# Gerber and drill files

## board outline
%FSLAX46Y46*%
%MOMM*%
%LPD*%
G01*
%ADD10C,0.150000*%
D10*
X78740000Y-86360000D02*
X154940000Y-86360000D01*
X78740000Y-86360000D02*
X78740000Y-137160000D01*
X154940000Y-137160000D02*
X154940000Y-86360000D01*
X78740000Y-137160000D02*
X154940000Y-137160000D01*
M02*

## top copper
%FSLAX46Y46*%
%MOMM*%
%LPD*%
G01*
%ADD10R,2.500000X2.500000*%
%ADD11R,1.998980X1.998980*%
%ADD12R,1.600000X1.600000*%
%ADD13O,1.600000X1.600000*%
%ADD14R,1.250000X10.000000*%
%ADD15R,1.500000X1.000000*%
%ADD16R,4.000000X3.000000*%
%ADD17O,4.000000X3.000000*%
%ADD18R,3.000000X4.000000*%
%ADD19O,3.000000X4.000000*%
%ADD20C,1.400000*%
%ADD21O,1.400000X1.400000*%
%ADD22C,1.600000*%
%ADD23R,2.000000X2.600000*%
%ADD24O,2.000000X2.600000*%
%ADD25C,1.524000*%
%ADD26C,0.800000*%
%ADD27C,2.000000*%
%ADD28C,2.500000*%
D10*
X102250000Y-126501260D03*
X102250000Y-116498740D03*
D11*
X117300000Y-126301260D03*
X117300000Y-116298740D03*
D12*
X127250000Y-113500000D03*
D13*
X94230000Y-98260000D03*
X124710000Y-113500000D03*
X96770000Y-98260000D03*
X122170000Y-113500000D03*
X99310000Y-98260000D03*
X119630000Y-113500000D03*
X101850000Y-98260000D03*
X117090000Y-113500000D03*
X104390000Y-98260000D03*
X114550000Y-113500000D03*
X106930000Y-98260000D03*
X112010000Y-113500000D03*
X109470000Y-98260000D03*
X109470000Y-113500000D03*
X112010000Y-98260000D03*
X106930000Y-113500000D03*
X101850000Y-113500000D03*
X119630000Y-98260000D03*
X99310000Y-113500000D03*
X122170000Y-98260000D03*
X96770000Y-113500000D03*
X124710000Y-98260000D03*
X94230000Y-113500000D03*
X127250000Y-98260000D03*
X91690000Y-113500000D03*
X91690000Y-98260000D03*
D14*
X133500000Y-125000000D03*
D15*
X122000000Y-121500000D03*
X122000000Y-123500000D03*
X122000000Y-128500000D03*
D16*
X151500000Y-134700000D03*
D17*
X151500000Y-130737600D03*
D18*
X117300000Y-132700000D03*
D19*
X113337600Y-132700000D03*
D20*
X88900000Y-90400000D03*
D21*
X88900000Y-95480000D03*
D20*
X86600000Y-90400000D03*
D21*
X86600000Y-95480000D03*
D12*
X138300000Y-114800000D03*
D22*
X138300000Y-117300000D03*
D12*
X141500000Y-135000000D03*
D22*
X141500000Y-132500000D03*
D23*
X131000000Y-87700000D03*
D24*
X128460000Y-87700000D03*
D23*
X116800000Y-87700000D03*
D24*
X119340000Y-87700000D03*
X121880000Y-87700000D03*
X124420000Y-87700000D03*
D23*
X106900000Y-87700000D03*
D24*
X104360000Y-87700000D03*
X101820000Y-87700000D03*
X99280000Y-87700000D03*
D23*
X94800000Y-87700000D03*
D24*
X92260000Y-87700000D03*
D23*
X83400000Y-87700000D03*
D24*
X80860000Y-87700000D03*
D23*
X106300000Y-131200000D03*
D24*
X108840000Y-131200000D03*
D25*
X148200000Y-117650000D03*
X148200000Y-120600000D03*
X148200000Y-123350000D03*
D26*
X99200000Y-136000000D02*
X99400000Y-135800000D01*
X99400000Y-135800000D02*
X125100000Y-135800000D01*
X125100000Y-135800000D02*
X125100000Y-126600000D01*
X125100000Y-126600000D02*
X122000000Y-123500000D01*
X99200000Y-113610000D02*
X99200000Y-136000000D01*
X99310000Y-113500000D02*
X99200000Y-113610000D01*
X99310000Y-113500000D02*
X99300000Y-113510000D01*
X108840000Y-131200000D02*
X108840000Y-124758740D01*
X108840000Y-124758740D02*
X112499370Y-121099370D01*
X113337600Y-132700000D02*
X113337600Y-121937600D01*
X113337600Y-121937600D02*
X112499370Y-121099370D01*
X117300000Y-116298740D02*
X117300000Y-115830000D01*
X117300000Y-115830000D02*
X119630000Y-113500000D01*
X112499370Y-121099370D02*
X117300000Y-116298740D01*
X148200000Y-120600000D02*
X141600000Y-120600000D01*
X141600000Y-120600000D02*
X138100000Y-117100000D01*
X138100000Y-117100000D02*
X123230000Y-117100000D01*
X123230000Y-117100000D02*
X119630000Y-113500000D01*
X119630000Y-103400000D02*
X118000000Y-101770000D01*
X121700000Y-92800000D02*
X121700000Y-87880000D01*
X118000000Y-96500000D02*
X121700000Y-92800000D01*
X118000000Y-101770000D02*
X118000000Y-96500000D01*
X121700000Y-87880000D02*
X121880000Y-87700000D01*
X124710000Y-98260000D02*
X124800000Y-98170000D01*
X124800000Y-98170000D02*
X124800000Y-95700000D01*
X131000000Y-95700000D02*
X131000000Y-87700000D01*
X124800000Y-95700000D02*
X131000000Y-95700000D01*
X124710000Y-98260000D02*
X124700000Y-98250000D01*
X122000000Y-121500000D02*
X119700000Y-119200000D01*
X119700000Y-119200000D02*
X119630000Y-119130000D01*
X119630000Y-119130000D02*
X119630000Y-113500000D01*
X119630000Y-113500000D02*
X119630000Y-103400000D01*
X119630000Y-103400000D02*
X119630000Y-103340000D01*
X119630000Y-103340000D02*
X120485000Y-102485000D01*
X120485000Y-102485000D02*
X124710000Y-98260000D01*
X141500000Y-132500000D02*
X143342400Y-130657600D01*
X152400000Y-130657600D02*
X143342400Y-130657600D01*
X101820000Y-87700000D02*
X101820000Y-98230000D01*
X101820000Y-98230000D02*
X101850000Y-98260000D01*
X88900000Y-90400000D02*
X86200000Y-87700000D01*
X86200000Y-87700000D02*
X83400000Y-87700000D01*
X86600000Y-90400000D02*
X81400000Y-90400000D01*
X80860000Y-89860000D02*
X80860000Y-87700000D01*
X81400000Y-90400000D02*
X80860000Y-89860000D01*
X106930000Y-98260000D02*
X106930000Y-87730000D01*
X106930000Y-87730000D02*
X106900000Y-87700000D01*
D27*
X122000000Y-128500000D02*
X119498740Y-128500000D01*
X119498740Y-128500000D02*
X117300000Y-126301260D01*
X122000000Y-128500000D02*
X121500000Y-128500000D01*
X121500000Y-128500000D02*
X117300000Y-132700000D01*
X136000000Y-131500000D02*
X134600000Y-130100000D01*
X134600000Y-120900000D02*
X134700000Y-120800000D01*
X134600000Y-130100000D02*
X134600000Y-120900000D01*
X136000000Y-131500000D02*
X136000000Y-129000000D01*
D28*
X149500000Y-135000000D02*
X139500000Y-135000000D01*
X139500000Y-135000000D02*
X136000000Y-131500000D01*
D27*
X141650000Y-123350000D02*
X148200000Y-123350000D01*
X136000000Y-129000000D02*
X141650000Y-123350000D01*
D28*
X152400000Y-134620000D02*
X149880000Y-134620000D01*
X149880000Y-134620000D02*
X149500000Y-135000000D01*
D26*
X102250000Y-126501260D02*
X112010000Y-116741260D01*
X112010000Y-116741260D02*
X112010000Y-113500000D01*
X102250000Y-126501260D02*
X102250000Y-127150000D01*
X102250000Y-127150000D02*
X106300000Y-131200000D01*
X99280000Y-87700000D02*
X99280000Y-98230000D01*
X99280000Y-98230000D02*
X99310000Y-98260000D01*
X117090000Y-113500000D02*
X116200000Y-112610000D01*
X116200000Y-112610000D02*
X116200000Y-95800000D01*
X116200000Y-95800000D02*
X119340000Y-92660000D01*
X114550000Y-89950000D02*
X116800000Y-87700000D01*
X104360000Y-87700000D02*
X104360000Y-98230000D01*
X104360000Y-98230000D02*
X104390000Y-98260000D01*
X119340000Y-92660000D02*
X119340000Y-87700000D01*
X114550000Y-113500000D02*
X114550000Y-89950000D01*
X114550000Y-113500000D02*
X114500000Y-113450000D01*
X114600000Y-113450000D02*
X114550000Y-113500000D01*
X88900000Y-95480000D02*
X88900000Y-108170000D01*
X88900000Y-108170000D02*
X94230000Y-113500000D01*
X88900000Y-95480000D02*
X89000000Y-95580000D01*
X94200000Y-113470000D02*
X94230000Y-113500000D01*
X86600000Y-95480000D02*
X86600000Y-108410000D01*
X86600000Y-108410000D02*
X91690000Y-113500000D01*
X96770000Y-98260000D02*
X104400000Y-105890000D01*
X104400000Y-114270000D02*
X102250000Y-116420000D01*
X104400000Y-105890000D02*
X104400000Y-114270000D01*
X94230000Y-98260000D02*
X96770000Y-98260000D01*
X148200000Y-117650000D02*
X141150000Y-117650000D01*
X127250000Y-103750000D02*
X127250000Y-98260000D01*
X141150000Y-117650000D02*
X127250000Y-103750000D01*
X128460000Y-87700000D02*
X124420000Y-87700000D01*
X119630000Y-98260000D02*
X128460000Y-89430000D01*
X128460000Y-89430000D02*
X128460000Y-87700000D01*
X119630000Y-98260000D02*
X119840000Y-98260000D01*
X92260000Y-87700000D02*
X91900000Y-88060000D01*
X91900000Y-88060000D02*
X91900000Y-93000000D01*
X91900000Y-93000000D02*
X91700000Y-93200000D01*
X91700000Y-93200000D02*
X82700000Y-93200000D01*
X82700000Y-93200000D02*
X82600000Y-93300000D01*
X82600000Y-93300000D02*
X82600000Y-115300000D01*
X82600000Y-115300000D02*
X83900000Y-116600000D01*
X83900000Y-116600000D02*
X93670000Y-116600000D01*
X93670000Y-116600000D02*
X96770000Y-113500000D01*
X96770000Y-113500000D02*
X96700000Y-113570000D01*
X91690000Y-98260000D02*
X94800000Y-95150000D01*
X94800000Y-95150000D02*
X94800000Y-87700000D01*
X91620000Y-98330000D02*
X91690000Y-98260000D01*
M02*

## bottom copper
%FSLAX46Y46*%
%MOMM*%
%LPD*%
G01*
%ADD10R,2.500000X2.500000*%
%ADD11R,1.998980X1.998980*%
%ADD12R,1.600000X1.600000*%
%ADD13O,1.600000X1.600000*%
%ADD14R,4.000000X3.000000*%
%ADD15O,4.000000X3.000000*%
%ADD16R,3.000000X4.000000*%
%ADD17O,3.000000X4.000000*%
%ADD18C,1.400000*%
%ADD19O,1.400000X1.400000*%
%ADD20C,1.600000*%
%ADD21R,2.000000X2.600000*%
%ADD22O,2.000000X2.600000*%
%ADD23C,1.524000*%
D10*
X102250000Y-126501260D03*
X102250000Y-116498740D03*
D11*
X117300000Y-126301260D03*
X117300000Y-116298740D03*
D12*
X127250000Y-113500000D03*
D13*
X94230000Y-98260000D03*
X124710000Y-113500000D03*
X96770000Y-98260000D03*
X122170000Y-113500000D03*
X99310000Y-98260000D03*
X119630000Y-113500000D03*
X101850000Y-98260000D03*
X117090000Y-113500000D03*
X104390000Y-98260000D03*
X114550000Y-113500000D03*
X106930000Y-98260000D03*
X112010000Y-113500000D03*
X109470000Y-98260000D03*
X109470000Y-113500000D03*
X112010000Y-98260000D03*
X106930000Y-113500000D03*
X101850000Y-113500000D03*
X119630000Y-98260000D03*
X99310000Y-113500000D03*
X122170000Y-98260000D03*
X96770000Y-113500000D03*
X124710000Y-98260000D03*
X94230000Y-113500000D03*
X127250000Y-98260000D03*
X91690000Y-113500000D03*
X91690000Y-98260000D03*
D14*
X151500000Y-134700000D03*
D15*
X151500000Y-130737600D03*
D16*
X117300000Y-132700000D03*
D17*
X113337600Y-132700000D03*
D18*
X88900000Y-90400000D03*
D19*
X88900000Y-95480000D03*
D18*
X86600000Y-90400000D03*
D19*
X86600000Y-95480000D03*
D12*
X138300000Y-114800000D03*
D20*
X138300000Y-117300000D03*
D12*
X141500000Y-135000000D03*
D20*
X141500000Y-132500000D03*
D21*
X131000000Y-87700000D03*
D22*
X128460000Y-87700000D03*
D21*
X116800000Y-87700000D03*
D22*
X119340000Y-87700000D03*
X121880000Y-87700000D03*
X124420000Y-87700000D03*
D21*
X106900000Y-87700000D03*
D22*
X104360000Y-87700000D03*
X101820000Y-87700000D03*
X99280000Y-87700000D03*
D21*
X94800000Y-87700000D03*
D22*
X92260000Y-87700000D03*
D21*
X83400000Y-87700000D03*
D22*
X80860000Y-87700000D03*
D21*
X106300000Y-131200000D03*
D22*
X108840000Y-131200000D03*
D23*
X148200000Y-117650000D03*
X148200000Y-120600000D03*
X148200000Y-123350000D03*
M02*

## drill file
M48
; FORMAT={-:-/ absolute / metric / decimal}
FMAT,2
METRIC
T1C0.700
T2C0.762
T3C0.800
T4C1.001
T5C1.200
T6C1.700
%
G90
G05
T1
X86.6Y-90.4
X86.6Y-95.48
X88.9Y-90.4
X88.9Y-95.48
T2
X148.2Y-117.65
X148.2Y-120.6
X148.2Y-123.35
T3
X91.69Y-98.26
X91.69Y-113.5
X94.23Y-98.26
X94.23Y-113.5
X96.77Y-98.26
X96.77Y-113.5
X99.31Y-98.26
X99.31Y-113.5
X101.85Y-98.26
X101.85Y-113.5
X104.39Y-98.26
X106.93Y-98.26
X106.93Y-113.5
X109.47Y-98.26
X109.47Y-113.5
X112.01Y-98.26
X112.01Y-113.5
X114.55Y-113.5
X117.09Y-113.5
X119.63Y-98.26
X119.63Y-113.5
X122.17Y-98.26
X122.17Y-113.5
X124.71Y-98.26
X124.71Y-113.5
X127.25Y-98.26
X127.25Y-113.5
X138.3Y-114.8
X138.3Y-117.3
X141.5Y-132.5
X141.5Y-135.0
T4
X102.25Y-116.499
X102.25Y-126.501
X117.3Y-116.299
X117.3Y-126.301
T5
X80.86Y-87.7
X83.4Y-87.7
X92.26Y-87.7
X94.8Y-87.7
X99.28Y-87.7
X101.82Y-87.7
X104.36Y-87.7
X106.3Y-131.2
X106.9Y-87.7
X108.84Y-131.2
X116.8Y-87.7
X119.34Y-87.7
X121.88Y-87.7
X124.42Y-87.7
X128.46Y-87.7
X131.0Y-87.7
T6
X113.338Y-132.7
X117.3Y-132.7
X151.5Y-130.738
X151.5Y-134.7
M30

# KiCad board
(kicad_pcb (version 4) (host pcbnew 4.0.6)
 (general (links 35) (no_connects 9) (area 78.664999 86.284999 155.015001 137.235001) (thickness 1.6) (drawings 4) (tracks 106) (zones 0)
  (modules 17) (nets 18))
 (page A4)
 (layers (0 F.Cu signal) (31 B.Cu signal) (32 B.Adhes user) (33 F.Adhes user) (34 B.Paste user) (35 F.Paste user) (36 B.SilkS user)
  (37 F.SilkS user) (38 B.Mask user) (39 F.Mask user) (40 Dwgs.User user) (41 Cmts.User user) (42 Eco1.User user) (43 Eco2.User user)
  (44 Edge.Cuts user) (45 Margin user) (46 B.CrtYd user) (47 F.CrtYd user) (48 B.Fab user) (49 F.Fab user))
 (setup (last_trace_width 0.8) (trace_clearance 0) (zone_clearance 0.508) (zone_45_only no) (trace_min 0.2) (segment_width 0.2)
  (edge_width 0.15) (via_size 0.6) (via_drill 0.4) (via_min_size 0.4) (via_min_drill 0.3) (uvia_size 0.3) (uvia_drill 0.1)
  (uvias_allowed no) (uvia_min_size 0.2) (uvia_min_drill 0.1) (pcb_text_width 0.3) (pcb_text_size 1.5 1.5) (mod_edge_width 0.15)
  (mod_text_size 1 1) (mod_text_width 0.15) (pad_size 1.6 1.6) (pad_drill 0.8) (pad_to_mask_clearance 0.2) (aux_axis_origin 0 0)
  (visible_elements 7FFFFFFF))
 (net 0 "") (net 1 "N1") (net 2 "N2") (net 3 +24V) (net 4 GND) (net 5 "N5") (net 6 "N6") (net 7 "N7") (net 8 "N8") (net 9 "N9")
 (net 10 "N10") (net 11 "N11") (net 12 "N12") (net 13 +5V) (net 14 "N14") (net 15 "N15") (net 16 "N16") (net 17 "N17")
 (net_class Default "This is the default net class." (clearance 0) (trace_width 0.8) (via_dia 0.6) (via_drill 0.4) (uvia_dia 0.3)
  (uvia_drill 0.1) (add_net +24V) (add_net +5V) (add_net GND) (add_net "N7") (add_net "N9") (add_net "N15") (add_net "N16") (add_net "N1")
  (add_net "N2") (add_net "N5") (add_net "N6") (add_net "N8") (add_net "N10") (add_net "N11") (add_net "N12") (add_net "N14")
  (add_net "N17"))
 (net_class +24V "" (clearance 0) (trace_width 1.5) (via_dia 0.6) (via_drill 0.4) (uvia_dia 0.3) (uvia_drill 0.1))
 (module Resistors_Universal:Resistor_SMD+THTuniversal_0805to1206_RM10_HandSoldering (layer F.Cu) (at 102.25 121.5 90)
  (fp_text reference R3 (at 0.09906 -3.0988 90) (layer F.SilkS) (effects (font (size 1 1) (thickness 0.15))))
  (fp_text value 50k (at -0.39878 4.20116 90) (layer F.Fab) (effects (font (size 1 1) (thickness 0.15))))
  (pad 1 thru_hole rect (at -5.00126 0 270) (size 2.5 2.5) (drill 1.00076) (layers *.Cu *.Mask) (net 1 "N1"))
  (pad 2 thru_hole rect (at 5.00126 0 270) (size 2.5 2.5) (drill 1.00076) (layers *.Cu *.Mask) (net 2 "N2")))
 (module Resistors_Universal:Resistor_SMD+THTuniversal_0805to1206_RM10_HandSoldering (layer F.Cu) (at 117.3 121.3 90)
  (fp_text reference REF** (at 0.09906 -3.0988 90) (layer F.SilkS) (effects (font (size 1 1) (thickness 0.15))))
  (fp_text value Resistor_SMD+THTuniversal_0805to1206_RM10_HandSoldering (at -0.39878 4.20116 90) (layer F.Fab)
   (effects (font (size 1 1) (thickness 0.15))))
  (pad 1 thru_hole rect (at -5.00126 0 270) (size 1.99898 1.99898) (drill 1.00076) (layers *.Cu *.Mask) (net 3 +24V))
  (pad "" thru_hole rect (at 5.00126 0 270) (size 1.99898 1.99898) (drill 1.00076) (layers *.Cu *.Mask) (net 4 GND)))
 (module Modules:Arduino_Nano (layer B.Cu) (at 127.25 113.5 90)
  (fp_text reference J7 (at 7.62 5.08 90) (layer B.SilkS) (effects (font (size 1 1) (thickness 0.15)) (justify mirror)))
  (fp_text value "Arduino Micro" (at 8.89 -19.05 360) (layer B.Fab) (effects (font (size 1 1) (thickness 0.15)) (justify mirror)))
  (pad TX thru_hole rect (at 0 0 90) (size 1.6 1.6) (drill 0.8) (layers *.Cu *.Mask))
  (pad 3.3V thru_hole oval (at 15.24 -33.02 90) (size 1.6 1.6) (drill 0.8) (layers *.Cu *.Mask) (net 2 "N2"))
  (pad RX thru_hole oval (at 0 -2.54 90) (size 1.6 1.6) (drill 0.8) (layers *.Cu *.Mask))
  (pad AREF thru_hole oval (at 15.24 -30.48 90) (size 1.6 1.6) (drill 0.8) (layers *.Cu *.Mask) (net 2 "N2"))
  (pad RS thru_hole oval (at 0 -5.08 90) (size 1.6 1.6) (drill 0.8) (layers *.Cu *.Mask))
  (pad A0 thru_hole oval (at 15.24 -27.94 90) (size 1.6 1.6) (drill 0.8) (layers *.Cu *.Mask) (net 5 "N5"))
  (pad GND thru_hole oval (at 0 -7.62 90) (size 1.6 1.6) (drill 0.8) (layers *.Cu *.Mask) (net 4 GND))
  (pad A1 thru_hole oval (at 15.24 -25.4 90) (size 1.6 1.6) (drill 0.8) (layers *.Cu *.Mask) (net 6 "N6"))
  (pad SDA thru_hole oval (at 0 -10.16 90) (size 1.6 1.6) (drill 0.8) (layers *.Cu *.Mask) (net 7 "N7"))
  (pad A2 thru_hole oval (at 15.24 -22.86 90) (size 1.6 1.6) (drill 0.8) (layers *.Cu *.Mask) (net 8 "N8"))
  (pad SCL thru_hole oval (at 0 -12.7 90) (size 1.6 1.6) (drill 0.8) (layers *.Cu *.Mask) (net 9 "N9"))
  (pad A3 thru_hole oval (at 15.24 -20.32 90) (size 1.6 1.6) (drill 0.8) (layers *.Cu *.Mask) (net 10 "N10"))
  (pad D4 thru_hole oval (at 0 -15.24 90) (size 1.6 1.6) (drill 0.8) (layers *.Cu *.Mask) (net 1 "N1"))
  (pad A4 thru_hole oval (at 15.24 -17.78 90) (size 1.6 1.6) (drill 0.8) (layers *.Cu *.Mask))
  (pad D5 thru_hole oval (at 0 -17.78 90) (size 1.6 1.6) (drill 0.8) (layers *.Cu *.Mask))
  (pad A5 thru_hole oval (at 15.24 -15.24 90) (size 1.6 1.6) (drill 0.8) (layers *.Cu *.Mask) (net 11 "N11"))
  (pad D6 thru_hole oval (at 0 -20.32 90) (size 1.6 1.6) (drill 0.8) (layers *.Cu *.Mask))
  (pad D8 thru_hole oval (at 0 -25.4 90) (size 1.6 1.6) (drill 0.8) (layers *.Cu *.Mask))
  (pad 5v thru_hole oval (at 15.24 -7.62 90) (size 1.6 1.6) (drill 0.8) (layers *.Cu *.Mask))
  (pad D9 thru_hole oval (at 0 -27.94 90) (size 1.6 1.6) (drill 0.8) (layers *.Cu *.Mask))
  (pad RS thru_hole oval (at 15.24 -5.08 90) (size 1.6 1.6) (drill 0.8) (layers *.Cu *.Mask))
  (pad D10 thru_hole oval (at 0 -30.48 90) (size 1.6 1.6) (drill 0.8) (layers *.Cu *.Mask))
  (pad GND thru_hole oval (at 15.24 -2.54 90) (size 1.6 1.6) (drill 0.8) (layers *.Cu *.Mask) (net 4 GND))
  (pad D11 thru_hole oval (at 0 -33.02 90) (size 1.6 1.6) (drill 0.8) (layers *.Cu *.Mask) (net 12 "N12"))
  (pad Vin thru_hole oval (at 15.24 0 90) (size 1.6 1.6) (drill 0.8) (layers *.Cu *.Mask) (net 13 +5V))
  (pad D12 thru_hole oval (at 0 -35.56 90) (size 1.6 1.6) (drill 0.8) (layers *.Cu *.Mask) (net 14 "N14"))
  (pad D13 thru_hole oval (at 15.24 -35.56 90) (size 1.6 1.6) (drill 0.8) (layers *.Cu *.Mask)))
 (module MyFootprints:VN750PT (layer F.Cu) (at 128 125 270)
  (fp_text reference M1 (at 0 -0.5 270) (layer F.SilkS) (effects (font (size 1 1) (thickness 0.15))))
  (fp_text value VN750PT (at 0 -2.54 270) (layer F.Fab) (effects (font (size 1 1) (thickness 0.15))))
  (pad Vcc smd rect (at 0 -5.5 270) (size 10 1.25) (layers F.Cu F.Paste F.Mask) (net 3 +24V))
  (pad GND smd rect (at -3.5 6 270) (size 1 1.5) (layers F.Cu F.Paste F.Mask))
  (pad Inpu smd rect (at -1.5 6 270) (size 1 1.5) (layers F.Cu F.Paste F.Mask))
  (pad Vout smd rect (at 3.5 6 270) (size 1 1.5) (layers F.Cu F.Paste F.Mask) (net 3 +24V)))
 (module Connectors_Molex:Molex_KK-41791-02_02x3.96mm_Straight (layer F.Cu) (at 151.5 134.7 90)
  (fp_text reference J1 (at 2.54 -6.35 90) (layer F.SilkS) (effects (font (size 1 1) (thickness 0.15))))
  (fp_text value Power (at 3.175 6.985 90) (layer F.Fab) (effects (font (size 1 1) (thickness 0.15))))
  (pad 1 thru_hole rect (at 0 0 90) (size 3 4) (drill 1.7) (layers *.Cu *.Mask) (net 3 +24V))
  (pad 2 thru_hole oval (at 3.9624 0 90) (size 3 4) (drill 1.7) (layers *.Cu *.Mask) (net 4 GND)))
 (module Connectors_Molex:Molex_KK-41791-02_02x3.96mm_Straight (layer B.Cu) (at 117.3 132.7 180)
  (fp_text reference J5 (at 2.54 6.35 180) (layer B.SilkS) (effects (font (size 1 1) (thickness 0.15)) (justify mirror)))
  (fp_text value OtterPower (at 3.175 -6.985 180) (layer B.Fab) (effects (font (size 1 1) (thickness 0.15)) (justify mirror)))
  (pad 1 thru_hole rect (at 0 0 180) (size 3 4) (drill 1.7) (layers *.Cu *.Mask) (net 3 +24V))
  (pad 2 thru_hole oval (at 3.9624 0 180) (size 3 4) (drill 1.7) (layers *.Cu *.Mask) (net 4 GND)))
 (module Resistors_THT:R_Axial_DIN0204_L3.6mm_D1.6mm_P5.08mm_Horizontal (layer F.Cu) (at 88.9 90.4 270)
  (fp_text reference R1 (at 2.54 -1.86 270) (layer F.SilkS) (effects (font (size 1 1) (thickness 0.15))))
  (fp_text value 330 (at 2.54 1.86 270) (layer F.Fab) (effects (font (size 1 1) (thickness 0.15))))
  (pad 1 thru_hole circle (at 0 0 270) (size 1.4 1.4) (drill 0.7) (layers *.Cu *.Mask) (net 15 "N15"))
  (pad 2 thru_hole oval (at 5.08 0 270) (size 1.4 1.4) (drill 0.7) (layers *.Cu *.Mask) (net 12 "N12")))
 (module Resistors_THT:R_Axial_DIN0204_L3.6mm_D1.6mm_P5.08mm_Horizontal (layer F.Cu) (at 86.6 90.4 270)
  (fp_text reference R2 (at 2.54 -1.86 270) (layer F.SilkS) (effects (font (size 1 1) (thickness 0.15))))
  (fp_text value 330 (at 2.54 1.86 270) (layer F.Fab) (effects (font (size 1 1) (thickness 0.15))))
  (pad 1 thru_hole circle (at 0 0 270) (size 1.4 1.4) (drill 0.7) (layers *.Cu *.Mask) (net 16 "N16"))
  (pad 2 thru_hole oval (at 5.08 0 270) (size 1.4 1.4) (drill 0.7) (layers *.Cu *.Mask) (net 14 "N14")))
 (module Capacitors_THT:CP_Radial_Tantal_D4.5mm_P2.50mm (layer B.Cu) (at 138.3 114.8 270)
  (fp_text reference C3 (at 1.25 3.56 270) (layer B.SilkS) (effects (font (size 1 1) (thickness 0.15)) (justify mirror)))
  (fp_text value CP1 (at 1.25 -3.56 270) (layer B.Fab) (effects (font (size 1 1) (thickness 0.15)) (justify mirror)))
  (pad + thru_hole rect (at 0 0 270) (size 1.6 1.6) (drill 0.8) (layers *.Cu *.Mask) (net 13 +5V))
  (pad 2 thru_hole circle (at 2.5 0 270) (size 1.6 1.6) (drill 0.8) (layers *.Cu *.Mask) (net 4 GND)))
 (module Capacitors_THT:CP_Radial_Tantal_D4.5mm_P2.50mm (layer B.Cu) (at 141.5 135 90)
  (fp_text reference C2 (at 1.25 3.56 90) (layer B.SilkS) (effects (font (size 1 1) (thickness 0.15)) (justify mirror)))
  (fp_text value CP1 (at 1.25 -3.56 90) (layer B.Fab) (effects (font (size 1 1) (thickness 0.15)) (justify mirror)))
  (pad 1 thru_hole rect (at 0 0 90) (size 1.6 1.6) (drill 0.8) (layers *.Cu *.Mask) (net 3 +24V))
  (pad 2 thru_hole circle (at 2.5 0 90) (size 1.6 1.6) (drill 0.8) (layers *.Cu *.Mask) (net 4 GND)))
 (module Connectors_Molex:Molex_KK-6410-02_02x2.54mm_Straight (layer F.Cu) (at 131 87.7 180)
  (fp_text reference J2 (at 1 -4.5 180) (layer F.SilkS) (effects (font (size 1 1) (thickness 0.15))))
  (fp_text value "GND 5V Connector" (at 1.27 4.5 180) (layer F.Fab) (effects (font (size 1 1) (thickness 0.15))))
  (pad 1 thru_hole rect (at 0 0 180) (size 2 2.6) (drill 1.2) (layers *.Cu *.Mask) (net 4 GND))
  (pad 2 thru_hole oval (at 2.54 0 180) (size 2 2.6) (drill 1.2) (layers *.Cu *.Mask) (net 13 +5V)))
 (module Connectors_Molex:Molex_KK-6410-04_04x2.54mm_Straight (layer B.Cu) (at 116.8 87.7)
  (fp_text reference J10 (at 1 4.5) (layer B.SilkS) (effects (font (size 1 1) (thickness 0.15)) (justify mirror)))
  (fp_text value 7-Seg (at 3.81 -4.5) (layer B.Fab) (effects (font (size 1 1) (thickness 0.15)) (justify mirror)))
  (pad 1 thru_hole rect (at 0 0) (size 2 2.6) (drill 1.2) (layers *.Cu *.Mask) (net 7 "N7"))
  (pad 2 thru_hole oval (at 2.54 0) (size 2 2.6) (drill 1.2) (layers *.Cu *.Mask) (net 9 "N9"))
  (pad 3 thru_hole oval (at 5.08 0) (size 2 2.6) (drill 1.2) (layers *.Cu *.Mask) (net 4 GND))
  (pad 4 thru_hole oval (at 7.62 0) (size 2 2.6) (drill 1.2) (layers *.Cu *.Mask) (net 13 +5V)))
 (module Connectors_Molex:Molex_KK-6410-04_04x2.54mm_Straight (layer F.Cu) (at 106.9 87.7 180)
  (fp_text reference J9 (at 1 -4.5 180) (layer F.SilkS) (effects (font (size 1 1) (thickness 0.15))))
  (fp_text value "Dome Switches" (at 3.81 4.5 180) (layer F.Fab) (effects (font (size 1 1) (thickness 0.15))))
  (pad 1 thru_hole rect (at 0 0 180) (size 2 2.6) (drill 1.2) (layers *.Cu *.Mask) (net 10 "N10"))
  (pad 2 thru_hole oval (at 2.54 0 180) (size 2 2.6) (drill 1.2) (layers *.Cu *.Mask) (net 8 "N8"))
  (pad 3 thru_hole oval (at 5.08 0 180) (size 2 2.6) (drill 1.2) (layers *.Cu *.Mask) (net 6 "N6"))
  (pad 4 thru_hole oval (at 7.62 0 180) (size 2 2.6) (drill 1.2) (layers *.Cu *.Mask) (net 5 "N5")))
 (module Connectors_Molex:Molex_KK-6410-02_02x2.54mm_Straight (layer F.Cu) (at 94.8 87.7 180)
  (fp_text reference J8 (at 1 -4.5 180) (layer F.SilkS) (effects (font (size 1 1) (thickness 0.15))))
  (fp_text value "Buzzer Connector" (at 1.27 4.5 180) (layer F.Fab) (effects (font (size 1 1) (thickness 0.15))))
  (pad 1 thru_hole rect (at 0 0 180) (size 2 2.6) (drill 1.2) (layers *.Cu *.Mask) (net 11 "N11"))
  (pad 2 thru_hole oval (at 2.54 0 180) (size 2 2.6) (drill 1.2) (layers *.Cu *.Mask) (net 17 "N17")))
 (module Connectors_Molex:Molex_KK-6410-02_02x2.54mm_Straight (layer F.Cu) (at 83.4 87.7 180)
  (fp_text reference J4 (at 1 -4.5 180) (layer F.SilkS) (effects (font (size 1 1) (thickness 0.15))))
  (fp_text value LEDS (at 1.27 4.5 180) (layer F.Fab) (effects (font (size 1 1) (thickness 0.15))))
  (pad 1 thru_hole rect (at 0 0 180) (size 2 2.6) (drill 1.2) (layers *.Cu *.Mask) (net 15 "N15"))
  (pad 2 thru_hole oval (at 2.54 0 180) (size 2 2.6) (drill 1.2) (layers *.Cu *.Mask) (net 16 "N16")))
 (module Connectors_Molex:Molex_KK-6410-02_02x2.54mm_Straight (layer F.Cu) (at 106.3 131.2)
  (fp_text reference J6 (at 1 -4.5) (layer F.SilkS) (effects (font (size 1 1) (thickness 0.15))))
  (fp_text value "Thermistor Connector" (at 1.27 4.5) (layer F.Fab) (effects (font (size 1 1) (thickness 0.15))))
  (pad 1 thru_hole rect (at 0 0) (size 2 2.6) (drill 1.2) (layers *.Cu *.Mask) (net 1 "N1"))
  (pad 2 thru_hole oval (at 2.54 0) (size 2 2.6) (drill 1.2) (layers *.Cu *.Mask) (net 4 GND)))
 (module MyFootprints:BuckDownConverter (layer F.Cu) (at 146.2 120.6 270)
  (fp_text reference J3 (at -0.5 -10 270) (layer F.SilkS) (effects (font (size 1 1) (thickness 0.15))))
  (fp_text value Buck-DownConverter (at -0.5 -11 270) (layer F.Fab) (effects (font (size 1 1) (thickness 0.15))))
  (pad Vout thru_hole circle (at -2.95 -2 270) (size 1.524 1.524) (drill 0.762) (layers *.Cu *.Mask) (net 13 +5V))
  (pad GND thru_hole circle (at 0 -2 270) (size 1.524 1.524) (drill 0.762) (layers *.Cu *.Mask) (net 4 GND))
  (pad Vin thru_hole circle (at 2.75 -2 270) (size 1.524 1.524) (drill 0.762) (layers *.Cu *.Mask) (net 3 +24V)))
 (gr_line (start 78.74 86.36) (end 154.94 86.36) (angle 90) (layer Edge.Cuts) (width 0.15))
 (gr_line (start 78.74 86.36) (end 78.74 137.16) (angle 90) (layer Edge.Cuts) (width 0.15))
 (gr_line (start 154.94 137.16) (end 154.94 86.36) (angle 90) (layer Edge.Cuts) (width 0.15))
 (gr_line (start 78.74 137.16) (end 154.94 137.16) (angle 90) (layer Edge.Cuts) (width 0.15))
 (segment (start 99.2 136) (end 99.4 135.8) (width 0.8) (layer F.Cu) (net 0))
 (segment (start 99.4 135.8) (end 125.1 135.8) (width 0.8) (layer F.Cu) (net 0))
 (segment (start 125.1 135.8) (end 125.1 126.6) (width 0.8) (layer F.Cu) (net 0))
 (segment (start 125.1 126.6) (end 122 123.5) (width 0.8) (layer F.Cu) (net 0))
 (segment (start 99.2 113.61) (end 99.2 136) (width 0.8) (layer F.Cu) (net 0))
 (segment (start 99.31 113.5) (end 99.2 113.61) (width 0.8) (layer F.Cu) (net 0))
 (segment (start 99.31 113.5) (end 99.3 113.51) (width 0.8) (layer F.Cu) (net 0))
 (segment (start 108.84 131.2) (end 108.84 124.75874) (width 0.8) (layer F.Cu) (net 4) (status 400000))
 (segment (start 108.84 124.75874) (end 112.49937 121.09937) (width 0.8) (layer F.Cu) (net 4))
 (segment (start 113.3376 132.7) (end 113.3376 121.9376) (width 0.8) (layer F.Cu) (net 4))
 (segment (start 113.3376 121.9376) (end 112.49937 121.09937) (width 0.8) (layer F.Cu) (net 4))
 (segment (start 117.3 116.29874) (end 117.3 115.83) (width 0.8) (layer F.Cu) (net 4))
 (segment (start 117.3 115.83) (end 119.63 113.5) (width 0.8) (layer F.Cu) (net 4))
 (segment (start 112.49937 121.09937) (end 117.3 116.29874) (width 0.8) (layer F.Cu) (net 4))
 (segment (start 148.2 120.6) (end 141.6 120.6) (width 0.8) (layer F.Cu) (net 4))
 (segment (start 141.6 120.6) (end 138.1 117.1) (width 0.8) (layer F.Cu) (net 4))
 (segment (start 138.1 117.1) (end 123.23 117.1) (width 0.8) (layer F.Cu) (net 4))
 (segment (start 123.23 117.1) (end 119.63 113.5) (width 0.8) (layer F.Cu) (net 4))
 (segment (start 119.63 103.4) (end 118 101.77) (width 0.8) (layer F.Cu) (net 4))
 (segment (start 121.7 92.8) (end 121.7 87.88) (width 0.8) (layer F.Cu) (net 4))
 (segment (start 118 96.5) (end 121.7 92.8) (width 0.8) (layer F.Cu) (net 4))
 (segment (start 118 101.77) (end 118 96.5) (width 0.8) (layer F.Cu) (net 4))
 (segment (start 121.7 87.88) (end 121.88 87.7) (width 0.8) (layer F.Cu) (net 4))
 (segment (start 124.71 98.26) (end 124.8 98.17) (width 0.8) (layer F.Cu) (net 4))
 (segment (start 124.8 98.17) (end 124.8 95.7) (width 0.8) (layer F.Cu) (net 4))
 (segment (start 131 95.7) (end 131 87.7) (width 0.8) (layer F.Cu) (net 4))
 (segment (start 124.8 95.7) (end 131 95.7) (width 0.8) (layer F.Cu) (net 4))
 (segment (start 124.71 98.26) (end 124.7 98.25) (width 0.8) (layer F.Cu) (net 4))
 (segment (start 122 121.5) (end 119.7 119.2) (width 0.8) (layer F.Cu) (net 4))
 (segment (start 119.7 119.2) (end 119.63 119.13) (width 0.8) (layer F.Cu) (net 4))
 (segment (start 119.63 119.13) (end 119.63 113.5) (width 0.8) (layer F.Cu) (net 4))
 (segment (start 119.63 113.5) (end 119.63 103.4) (width 0.8) (layer F.Cu) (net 4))
 (segment (start 119.63 103.4) (end 119.63 103.34) (width 0.8) (layer F.Cu) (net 4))
 (segment (start 119.63 103.34) (end 120.485 102.485) (width 0.8) (layer F.Cu) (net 4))
 (segment (start 120.485 102.485) (end 124.71 98.26) (width 0.8) (layer F.Cu) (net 4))
 (segment (start 141.5 132.5) (end 143.3424 130.6576) (width 0.8) (layer F.Cu) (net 4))
 (segment (start 152.4 130.6576) (end 143.3424 130.6576) (width 0.8) (layer F.Cu) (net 4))
 (segment (start 101.82 87.7) (end 101.82 98.23) (width 0.8) (layer F.Cu) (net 6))
 (segment (start 101.82 98.23) (end 101.85 98.26) (width 0.8) (layer F.Cu) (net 6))
 (segment (start 88.9 90.4) (end 86.2 87.7) (width 0.8) (layer F.Cu) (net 15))
 (segment (start 86.2 87.7) (end 83.4 87.7) (width 0.8) (layer F.Cu) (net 15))
 (segment (start 86.6 90.4) (end 81.4 90.4) (width 0.8) (layer F.Cu) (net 16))
 (segment (start 80.86 89.86) (end 80.86 87.7) (width 0.8) (layer F.Cu) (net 16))
 (segment (start 81.4 90.4) (end 80.86 89.86) (width 0.8) (layer F.Cu) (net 16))
 (segment (start 106.93 98.26) (end 106.93 87.73) (width 0.8) (layer F.Cu) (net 10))
 (segment (start 106.93 87.73) (end 106.9 87.7) (width 0.8) (layer F.Cu) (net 10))
 (segment (start 122 128.5) (end 119.49874 128.5) (width 2) (layer F.Cu) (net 3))
 (segment (start 119.49874 128.5) (end 117.3 126.30126) (width 2) (layer F.Cu) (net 3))
 (segment (start 122 128.5) (end 121.5 128.5) (width 2) (layer F.Cu) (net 3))
 (segment (start 121.5 128.5) (end 117.3 132.7) (width 2) (layer F.Cu) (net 3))
 (segment (start 136 131.5) (end 134.6 130.1) (width 2) (layer F.Cu) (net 3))
 (segment (start 134.6 120.9) (end 134.7 120.8) (width 2) (layer F.Cu) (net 3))
 (segment (start 134.6 130.1) (end 134.6 120.9) (width 2) (layer F.Cu) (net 3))
 (segment (start 136 131.5) (end 136 129) (width 2) (layer F.Cu) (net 3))
 (segment (start 149.5 135) (end 139.5 135) (width 2.5) (layer F.Cu) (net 3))
 (segment (start 139.5 135) (end 136 131.5) (width 2.5) (layer F.Cu) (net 3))
 (segment (start 141.65 123.35) (end 148.2 123.35) (width 2) (layer F.Cu) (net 3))
 (segment (start 136 129) (end 141.65 123.35) (width 2) (layer F.Cu) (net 3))
 (segment (start 152.4 134.62) (end 149.88 134.62) (width 2.5) (layer F.Cu) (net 3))
 (segment (start 149.88 134.62) (end 149.5 135) (width 2.5) (layer F.Cu) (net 3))
 (segment (start 102.25 126.50126) (end 112.01 116.74126) (width 0.8) (layer F.Cu) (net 1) (status 400000))
 (segment (start 112.01 116.74126) (end 112.01 113.5) (width 0.8) (layer F.Cu) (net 1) (status 800000))
 (segment (start 102.25 126.50126) (end 102.25 127.15) (width 0.8) (layer F.Cu) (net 1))
 (segment (start 102.25 127.15) (end 106.3 131.2) (width 0.8) (layer F.Cu) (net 1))
 (segment (start 99.28 87.7) (end 99.28 98.23) (width 0.8) (layer F.Cu) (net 5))
 (segment (start 99.28 98.23) (end 99.31 98.26) (width 0.8) (layer F.Cu) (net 5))
 (segment (start 117.09 113.5) (end 116.2 112.61) (width 0.8) (layer F.Cu) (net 7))
 (segment (start 116.2 112.61) (end 116.2 95.8) (width 0.8) (layer F.Cu) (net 7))
 (segment (start 116.2 95.8) (end 119.34 92.66) (width 0.8) (layer F.Cu) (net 7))
 (segment (start 114.55 89.95) (end 116.8 87.7) (width 0.8) (layer F.Cu) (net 7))
 (segment (start 104.36 87.7) (end 104.36 98.23) (width 0.8) (layer F.Cu) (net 8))
 (segment (start 104.36 98.23) (end 104.39 98.26) (width 0.8) (layer F.Cu) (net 8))
 (segment (start 119.34 92.66) (end 119.34 87.7) (width 0.8) (layer F.Cu) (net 9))
 (segment (start 114.55 113.5) (end 114.55 89.95) (width 0.8) (layer F.Cu) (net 9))
 (segment (start 114.55 113.5) (end 114.5 113.45) (width 0.8) (layer F.Cu) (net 9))
 (segment (start 114.6 113.45) (end 114.55 113.5) (width 0.8) (layer F.Cu) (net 9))
 (segment (start 88.9 95.48) (end 88.9 108.17) (width 0.8) (layer F.Cu) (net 12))
 (segment (start 88.9 108.17) (end 94.23 113.5) (width 0.8) (layer F.Cu) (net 12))
 (segment (start 88.9 95.48) (end 89 95.58) (width 0.8) (layer F.Cu) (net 12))
 (segment (start 94.2 113.47) (end 94.23 113.5) (width 0.8) (layer F.Cu) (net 12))
 (segment (start 86.6 95.48) (end 86.6 108.41) (width 0.8) (layer F.Cu) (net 14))
 (segment (start 86.6 108.41) (end 91.69 113.5) (width 0.8) (layer F.Cu) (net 14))
 (segment (start 96.77 98.26) (end 104.4 105.89) (width 0.8) (layer F.Cu) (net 2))
 (segment (start 104.4 114.27) (end 102.25 116.42) (width 0.8) (layer F.Cu) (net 2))
 (segment (start 104.4 105.89) (end 104.4 114.27) (width 0.8) (layer F.Cu) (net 2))
 (segment (start 94.23 98.26) (end 96.77 98.26) (width 0.8) (layer F.Cu) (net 2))
 (segment (start 148.2 117.65) (end 141.15 117.65) (width 0.8) (layer F.Cu) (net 13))
 (segment (start 127.25 103.75) (end 127.25 98.26) (width 0.8) (layer F.Cu) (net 13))
 (segment (start 141.15 117.65) (end 127.25 103.75) (width 0.8) (layer F.Cu) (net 13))
 (segment (start 128.46 87.7) (end 124.42 87.7) (width 0.8) (layer F.Cu) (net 13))
 (segment (start 119.63 98.26) (end 128.46 89.43) (width 0.8) (layer F.Cu) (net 13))
 (segment (start 128.46 89.43) (end 128.46 87.7) (width 0.8) (layer F.Cu) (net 13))
 (segment (start 119.63 98.26) (end 119.84 98.26) (width 0.8) (layer F.Cu) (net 13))
 (segment (start 92.26 87.7) (end 91.9 88.06) (width 0.8) (layer F.Cu) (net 17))
 (segment (start 91.9 88.06) (end 91.9 93) (width 0.8) (layer F.Cu) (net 17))
 (segment (start 91.9 93) (end 91.7 93.2) (width 0.8) (layer F.Cu) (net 17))
 (segment (start 91.7 93.2) (end 82.7 93.2) (width 0.8) (layer F.Cu) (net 17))
 (segment (start 82.7 93.2) (end 82.6 93.3) (width 0.8) (layer F.Cu) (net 17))
 (segment (start 82.6 93.3) (end 82.6 115.3) (width 0.8) (layer F.Cu) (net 17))
 (segment (start 82.6 115.3) (end 83.9 116.6) (width 0.8) (layer F.Cu) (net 17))
 (segment (start 83.9 116.6) (end 93.67 116.6) (width 0.8) (layer F.Cu) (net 17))
 (segment (start 93.67 116.6) (end 96.77 113.5) (width 0.8) (layer F.Cu) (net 17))
 (segment (start 96.77 113.5) (end 96.7 113.57) (width 0.8) (layer F.Cu) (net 17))
 (segment (start 91.69 98.26) (end 94.8 95.15) (width 0.8) (layer F.Cu) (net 11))
 (segment (start 94.8 95.15) (end 94.8 87.7) (width 0.8) (layer F.Cu) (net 11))
 (segment (start 91.62 98.33) (end 91.69 98.26) (width 0.8) (layer F.Cu) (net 11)))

